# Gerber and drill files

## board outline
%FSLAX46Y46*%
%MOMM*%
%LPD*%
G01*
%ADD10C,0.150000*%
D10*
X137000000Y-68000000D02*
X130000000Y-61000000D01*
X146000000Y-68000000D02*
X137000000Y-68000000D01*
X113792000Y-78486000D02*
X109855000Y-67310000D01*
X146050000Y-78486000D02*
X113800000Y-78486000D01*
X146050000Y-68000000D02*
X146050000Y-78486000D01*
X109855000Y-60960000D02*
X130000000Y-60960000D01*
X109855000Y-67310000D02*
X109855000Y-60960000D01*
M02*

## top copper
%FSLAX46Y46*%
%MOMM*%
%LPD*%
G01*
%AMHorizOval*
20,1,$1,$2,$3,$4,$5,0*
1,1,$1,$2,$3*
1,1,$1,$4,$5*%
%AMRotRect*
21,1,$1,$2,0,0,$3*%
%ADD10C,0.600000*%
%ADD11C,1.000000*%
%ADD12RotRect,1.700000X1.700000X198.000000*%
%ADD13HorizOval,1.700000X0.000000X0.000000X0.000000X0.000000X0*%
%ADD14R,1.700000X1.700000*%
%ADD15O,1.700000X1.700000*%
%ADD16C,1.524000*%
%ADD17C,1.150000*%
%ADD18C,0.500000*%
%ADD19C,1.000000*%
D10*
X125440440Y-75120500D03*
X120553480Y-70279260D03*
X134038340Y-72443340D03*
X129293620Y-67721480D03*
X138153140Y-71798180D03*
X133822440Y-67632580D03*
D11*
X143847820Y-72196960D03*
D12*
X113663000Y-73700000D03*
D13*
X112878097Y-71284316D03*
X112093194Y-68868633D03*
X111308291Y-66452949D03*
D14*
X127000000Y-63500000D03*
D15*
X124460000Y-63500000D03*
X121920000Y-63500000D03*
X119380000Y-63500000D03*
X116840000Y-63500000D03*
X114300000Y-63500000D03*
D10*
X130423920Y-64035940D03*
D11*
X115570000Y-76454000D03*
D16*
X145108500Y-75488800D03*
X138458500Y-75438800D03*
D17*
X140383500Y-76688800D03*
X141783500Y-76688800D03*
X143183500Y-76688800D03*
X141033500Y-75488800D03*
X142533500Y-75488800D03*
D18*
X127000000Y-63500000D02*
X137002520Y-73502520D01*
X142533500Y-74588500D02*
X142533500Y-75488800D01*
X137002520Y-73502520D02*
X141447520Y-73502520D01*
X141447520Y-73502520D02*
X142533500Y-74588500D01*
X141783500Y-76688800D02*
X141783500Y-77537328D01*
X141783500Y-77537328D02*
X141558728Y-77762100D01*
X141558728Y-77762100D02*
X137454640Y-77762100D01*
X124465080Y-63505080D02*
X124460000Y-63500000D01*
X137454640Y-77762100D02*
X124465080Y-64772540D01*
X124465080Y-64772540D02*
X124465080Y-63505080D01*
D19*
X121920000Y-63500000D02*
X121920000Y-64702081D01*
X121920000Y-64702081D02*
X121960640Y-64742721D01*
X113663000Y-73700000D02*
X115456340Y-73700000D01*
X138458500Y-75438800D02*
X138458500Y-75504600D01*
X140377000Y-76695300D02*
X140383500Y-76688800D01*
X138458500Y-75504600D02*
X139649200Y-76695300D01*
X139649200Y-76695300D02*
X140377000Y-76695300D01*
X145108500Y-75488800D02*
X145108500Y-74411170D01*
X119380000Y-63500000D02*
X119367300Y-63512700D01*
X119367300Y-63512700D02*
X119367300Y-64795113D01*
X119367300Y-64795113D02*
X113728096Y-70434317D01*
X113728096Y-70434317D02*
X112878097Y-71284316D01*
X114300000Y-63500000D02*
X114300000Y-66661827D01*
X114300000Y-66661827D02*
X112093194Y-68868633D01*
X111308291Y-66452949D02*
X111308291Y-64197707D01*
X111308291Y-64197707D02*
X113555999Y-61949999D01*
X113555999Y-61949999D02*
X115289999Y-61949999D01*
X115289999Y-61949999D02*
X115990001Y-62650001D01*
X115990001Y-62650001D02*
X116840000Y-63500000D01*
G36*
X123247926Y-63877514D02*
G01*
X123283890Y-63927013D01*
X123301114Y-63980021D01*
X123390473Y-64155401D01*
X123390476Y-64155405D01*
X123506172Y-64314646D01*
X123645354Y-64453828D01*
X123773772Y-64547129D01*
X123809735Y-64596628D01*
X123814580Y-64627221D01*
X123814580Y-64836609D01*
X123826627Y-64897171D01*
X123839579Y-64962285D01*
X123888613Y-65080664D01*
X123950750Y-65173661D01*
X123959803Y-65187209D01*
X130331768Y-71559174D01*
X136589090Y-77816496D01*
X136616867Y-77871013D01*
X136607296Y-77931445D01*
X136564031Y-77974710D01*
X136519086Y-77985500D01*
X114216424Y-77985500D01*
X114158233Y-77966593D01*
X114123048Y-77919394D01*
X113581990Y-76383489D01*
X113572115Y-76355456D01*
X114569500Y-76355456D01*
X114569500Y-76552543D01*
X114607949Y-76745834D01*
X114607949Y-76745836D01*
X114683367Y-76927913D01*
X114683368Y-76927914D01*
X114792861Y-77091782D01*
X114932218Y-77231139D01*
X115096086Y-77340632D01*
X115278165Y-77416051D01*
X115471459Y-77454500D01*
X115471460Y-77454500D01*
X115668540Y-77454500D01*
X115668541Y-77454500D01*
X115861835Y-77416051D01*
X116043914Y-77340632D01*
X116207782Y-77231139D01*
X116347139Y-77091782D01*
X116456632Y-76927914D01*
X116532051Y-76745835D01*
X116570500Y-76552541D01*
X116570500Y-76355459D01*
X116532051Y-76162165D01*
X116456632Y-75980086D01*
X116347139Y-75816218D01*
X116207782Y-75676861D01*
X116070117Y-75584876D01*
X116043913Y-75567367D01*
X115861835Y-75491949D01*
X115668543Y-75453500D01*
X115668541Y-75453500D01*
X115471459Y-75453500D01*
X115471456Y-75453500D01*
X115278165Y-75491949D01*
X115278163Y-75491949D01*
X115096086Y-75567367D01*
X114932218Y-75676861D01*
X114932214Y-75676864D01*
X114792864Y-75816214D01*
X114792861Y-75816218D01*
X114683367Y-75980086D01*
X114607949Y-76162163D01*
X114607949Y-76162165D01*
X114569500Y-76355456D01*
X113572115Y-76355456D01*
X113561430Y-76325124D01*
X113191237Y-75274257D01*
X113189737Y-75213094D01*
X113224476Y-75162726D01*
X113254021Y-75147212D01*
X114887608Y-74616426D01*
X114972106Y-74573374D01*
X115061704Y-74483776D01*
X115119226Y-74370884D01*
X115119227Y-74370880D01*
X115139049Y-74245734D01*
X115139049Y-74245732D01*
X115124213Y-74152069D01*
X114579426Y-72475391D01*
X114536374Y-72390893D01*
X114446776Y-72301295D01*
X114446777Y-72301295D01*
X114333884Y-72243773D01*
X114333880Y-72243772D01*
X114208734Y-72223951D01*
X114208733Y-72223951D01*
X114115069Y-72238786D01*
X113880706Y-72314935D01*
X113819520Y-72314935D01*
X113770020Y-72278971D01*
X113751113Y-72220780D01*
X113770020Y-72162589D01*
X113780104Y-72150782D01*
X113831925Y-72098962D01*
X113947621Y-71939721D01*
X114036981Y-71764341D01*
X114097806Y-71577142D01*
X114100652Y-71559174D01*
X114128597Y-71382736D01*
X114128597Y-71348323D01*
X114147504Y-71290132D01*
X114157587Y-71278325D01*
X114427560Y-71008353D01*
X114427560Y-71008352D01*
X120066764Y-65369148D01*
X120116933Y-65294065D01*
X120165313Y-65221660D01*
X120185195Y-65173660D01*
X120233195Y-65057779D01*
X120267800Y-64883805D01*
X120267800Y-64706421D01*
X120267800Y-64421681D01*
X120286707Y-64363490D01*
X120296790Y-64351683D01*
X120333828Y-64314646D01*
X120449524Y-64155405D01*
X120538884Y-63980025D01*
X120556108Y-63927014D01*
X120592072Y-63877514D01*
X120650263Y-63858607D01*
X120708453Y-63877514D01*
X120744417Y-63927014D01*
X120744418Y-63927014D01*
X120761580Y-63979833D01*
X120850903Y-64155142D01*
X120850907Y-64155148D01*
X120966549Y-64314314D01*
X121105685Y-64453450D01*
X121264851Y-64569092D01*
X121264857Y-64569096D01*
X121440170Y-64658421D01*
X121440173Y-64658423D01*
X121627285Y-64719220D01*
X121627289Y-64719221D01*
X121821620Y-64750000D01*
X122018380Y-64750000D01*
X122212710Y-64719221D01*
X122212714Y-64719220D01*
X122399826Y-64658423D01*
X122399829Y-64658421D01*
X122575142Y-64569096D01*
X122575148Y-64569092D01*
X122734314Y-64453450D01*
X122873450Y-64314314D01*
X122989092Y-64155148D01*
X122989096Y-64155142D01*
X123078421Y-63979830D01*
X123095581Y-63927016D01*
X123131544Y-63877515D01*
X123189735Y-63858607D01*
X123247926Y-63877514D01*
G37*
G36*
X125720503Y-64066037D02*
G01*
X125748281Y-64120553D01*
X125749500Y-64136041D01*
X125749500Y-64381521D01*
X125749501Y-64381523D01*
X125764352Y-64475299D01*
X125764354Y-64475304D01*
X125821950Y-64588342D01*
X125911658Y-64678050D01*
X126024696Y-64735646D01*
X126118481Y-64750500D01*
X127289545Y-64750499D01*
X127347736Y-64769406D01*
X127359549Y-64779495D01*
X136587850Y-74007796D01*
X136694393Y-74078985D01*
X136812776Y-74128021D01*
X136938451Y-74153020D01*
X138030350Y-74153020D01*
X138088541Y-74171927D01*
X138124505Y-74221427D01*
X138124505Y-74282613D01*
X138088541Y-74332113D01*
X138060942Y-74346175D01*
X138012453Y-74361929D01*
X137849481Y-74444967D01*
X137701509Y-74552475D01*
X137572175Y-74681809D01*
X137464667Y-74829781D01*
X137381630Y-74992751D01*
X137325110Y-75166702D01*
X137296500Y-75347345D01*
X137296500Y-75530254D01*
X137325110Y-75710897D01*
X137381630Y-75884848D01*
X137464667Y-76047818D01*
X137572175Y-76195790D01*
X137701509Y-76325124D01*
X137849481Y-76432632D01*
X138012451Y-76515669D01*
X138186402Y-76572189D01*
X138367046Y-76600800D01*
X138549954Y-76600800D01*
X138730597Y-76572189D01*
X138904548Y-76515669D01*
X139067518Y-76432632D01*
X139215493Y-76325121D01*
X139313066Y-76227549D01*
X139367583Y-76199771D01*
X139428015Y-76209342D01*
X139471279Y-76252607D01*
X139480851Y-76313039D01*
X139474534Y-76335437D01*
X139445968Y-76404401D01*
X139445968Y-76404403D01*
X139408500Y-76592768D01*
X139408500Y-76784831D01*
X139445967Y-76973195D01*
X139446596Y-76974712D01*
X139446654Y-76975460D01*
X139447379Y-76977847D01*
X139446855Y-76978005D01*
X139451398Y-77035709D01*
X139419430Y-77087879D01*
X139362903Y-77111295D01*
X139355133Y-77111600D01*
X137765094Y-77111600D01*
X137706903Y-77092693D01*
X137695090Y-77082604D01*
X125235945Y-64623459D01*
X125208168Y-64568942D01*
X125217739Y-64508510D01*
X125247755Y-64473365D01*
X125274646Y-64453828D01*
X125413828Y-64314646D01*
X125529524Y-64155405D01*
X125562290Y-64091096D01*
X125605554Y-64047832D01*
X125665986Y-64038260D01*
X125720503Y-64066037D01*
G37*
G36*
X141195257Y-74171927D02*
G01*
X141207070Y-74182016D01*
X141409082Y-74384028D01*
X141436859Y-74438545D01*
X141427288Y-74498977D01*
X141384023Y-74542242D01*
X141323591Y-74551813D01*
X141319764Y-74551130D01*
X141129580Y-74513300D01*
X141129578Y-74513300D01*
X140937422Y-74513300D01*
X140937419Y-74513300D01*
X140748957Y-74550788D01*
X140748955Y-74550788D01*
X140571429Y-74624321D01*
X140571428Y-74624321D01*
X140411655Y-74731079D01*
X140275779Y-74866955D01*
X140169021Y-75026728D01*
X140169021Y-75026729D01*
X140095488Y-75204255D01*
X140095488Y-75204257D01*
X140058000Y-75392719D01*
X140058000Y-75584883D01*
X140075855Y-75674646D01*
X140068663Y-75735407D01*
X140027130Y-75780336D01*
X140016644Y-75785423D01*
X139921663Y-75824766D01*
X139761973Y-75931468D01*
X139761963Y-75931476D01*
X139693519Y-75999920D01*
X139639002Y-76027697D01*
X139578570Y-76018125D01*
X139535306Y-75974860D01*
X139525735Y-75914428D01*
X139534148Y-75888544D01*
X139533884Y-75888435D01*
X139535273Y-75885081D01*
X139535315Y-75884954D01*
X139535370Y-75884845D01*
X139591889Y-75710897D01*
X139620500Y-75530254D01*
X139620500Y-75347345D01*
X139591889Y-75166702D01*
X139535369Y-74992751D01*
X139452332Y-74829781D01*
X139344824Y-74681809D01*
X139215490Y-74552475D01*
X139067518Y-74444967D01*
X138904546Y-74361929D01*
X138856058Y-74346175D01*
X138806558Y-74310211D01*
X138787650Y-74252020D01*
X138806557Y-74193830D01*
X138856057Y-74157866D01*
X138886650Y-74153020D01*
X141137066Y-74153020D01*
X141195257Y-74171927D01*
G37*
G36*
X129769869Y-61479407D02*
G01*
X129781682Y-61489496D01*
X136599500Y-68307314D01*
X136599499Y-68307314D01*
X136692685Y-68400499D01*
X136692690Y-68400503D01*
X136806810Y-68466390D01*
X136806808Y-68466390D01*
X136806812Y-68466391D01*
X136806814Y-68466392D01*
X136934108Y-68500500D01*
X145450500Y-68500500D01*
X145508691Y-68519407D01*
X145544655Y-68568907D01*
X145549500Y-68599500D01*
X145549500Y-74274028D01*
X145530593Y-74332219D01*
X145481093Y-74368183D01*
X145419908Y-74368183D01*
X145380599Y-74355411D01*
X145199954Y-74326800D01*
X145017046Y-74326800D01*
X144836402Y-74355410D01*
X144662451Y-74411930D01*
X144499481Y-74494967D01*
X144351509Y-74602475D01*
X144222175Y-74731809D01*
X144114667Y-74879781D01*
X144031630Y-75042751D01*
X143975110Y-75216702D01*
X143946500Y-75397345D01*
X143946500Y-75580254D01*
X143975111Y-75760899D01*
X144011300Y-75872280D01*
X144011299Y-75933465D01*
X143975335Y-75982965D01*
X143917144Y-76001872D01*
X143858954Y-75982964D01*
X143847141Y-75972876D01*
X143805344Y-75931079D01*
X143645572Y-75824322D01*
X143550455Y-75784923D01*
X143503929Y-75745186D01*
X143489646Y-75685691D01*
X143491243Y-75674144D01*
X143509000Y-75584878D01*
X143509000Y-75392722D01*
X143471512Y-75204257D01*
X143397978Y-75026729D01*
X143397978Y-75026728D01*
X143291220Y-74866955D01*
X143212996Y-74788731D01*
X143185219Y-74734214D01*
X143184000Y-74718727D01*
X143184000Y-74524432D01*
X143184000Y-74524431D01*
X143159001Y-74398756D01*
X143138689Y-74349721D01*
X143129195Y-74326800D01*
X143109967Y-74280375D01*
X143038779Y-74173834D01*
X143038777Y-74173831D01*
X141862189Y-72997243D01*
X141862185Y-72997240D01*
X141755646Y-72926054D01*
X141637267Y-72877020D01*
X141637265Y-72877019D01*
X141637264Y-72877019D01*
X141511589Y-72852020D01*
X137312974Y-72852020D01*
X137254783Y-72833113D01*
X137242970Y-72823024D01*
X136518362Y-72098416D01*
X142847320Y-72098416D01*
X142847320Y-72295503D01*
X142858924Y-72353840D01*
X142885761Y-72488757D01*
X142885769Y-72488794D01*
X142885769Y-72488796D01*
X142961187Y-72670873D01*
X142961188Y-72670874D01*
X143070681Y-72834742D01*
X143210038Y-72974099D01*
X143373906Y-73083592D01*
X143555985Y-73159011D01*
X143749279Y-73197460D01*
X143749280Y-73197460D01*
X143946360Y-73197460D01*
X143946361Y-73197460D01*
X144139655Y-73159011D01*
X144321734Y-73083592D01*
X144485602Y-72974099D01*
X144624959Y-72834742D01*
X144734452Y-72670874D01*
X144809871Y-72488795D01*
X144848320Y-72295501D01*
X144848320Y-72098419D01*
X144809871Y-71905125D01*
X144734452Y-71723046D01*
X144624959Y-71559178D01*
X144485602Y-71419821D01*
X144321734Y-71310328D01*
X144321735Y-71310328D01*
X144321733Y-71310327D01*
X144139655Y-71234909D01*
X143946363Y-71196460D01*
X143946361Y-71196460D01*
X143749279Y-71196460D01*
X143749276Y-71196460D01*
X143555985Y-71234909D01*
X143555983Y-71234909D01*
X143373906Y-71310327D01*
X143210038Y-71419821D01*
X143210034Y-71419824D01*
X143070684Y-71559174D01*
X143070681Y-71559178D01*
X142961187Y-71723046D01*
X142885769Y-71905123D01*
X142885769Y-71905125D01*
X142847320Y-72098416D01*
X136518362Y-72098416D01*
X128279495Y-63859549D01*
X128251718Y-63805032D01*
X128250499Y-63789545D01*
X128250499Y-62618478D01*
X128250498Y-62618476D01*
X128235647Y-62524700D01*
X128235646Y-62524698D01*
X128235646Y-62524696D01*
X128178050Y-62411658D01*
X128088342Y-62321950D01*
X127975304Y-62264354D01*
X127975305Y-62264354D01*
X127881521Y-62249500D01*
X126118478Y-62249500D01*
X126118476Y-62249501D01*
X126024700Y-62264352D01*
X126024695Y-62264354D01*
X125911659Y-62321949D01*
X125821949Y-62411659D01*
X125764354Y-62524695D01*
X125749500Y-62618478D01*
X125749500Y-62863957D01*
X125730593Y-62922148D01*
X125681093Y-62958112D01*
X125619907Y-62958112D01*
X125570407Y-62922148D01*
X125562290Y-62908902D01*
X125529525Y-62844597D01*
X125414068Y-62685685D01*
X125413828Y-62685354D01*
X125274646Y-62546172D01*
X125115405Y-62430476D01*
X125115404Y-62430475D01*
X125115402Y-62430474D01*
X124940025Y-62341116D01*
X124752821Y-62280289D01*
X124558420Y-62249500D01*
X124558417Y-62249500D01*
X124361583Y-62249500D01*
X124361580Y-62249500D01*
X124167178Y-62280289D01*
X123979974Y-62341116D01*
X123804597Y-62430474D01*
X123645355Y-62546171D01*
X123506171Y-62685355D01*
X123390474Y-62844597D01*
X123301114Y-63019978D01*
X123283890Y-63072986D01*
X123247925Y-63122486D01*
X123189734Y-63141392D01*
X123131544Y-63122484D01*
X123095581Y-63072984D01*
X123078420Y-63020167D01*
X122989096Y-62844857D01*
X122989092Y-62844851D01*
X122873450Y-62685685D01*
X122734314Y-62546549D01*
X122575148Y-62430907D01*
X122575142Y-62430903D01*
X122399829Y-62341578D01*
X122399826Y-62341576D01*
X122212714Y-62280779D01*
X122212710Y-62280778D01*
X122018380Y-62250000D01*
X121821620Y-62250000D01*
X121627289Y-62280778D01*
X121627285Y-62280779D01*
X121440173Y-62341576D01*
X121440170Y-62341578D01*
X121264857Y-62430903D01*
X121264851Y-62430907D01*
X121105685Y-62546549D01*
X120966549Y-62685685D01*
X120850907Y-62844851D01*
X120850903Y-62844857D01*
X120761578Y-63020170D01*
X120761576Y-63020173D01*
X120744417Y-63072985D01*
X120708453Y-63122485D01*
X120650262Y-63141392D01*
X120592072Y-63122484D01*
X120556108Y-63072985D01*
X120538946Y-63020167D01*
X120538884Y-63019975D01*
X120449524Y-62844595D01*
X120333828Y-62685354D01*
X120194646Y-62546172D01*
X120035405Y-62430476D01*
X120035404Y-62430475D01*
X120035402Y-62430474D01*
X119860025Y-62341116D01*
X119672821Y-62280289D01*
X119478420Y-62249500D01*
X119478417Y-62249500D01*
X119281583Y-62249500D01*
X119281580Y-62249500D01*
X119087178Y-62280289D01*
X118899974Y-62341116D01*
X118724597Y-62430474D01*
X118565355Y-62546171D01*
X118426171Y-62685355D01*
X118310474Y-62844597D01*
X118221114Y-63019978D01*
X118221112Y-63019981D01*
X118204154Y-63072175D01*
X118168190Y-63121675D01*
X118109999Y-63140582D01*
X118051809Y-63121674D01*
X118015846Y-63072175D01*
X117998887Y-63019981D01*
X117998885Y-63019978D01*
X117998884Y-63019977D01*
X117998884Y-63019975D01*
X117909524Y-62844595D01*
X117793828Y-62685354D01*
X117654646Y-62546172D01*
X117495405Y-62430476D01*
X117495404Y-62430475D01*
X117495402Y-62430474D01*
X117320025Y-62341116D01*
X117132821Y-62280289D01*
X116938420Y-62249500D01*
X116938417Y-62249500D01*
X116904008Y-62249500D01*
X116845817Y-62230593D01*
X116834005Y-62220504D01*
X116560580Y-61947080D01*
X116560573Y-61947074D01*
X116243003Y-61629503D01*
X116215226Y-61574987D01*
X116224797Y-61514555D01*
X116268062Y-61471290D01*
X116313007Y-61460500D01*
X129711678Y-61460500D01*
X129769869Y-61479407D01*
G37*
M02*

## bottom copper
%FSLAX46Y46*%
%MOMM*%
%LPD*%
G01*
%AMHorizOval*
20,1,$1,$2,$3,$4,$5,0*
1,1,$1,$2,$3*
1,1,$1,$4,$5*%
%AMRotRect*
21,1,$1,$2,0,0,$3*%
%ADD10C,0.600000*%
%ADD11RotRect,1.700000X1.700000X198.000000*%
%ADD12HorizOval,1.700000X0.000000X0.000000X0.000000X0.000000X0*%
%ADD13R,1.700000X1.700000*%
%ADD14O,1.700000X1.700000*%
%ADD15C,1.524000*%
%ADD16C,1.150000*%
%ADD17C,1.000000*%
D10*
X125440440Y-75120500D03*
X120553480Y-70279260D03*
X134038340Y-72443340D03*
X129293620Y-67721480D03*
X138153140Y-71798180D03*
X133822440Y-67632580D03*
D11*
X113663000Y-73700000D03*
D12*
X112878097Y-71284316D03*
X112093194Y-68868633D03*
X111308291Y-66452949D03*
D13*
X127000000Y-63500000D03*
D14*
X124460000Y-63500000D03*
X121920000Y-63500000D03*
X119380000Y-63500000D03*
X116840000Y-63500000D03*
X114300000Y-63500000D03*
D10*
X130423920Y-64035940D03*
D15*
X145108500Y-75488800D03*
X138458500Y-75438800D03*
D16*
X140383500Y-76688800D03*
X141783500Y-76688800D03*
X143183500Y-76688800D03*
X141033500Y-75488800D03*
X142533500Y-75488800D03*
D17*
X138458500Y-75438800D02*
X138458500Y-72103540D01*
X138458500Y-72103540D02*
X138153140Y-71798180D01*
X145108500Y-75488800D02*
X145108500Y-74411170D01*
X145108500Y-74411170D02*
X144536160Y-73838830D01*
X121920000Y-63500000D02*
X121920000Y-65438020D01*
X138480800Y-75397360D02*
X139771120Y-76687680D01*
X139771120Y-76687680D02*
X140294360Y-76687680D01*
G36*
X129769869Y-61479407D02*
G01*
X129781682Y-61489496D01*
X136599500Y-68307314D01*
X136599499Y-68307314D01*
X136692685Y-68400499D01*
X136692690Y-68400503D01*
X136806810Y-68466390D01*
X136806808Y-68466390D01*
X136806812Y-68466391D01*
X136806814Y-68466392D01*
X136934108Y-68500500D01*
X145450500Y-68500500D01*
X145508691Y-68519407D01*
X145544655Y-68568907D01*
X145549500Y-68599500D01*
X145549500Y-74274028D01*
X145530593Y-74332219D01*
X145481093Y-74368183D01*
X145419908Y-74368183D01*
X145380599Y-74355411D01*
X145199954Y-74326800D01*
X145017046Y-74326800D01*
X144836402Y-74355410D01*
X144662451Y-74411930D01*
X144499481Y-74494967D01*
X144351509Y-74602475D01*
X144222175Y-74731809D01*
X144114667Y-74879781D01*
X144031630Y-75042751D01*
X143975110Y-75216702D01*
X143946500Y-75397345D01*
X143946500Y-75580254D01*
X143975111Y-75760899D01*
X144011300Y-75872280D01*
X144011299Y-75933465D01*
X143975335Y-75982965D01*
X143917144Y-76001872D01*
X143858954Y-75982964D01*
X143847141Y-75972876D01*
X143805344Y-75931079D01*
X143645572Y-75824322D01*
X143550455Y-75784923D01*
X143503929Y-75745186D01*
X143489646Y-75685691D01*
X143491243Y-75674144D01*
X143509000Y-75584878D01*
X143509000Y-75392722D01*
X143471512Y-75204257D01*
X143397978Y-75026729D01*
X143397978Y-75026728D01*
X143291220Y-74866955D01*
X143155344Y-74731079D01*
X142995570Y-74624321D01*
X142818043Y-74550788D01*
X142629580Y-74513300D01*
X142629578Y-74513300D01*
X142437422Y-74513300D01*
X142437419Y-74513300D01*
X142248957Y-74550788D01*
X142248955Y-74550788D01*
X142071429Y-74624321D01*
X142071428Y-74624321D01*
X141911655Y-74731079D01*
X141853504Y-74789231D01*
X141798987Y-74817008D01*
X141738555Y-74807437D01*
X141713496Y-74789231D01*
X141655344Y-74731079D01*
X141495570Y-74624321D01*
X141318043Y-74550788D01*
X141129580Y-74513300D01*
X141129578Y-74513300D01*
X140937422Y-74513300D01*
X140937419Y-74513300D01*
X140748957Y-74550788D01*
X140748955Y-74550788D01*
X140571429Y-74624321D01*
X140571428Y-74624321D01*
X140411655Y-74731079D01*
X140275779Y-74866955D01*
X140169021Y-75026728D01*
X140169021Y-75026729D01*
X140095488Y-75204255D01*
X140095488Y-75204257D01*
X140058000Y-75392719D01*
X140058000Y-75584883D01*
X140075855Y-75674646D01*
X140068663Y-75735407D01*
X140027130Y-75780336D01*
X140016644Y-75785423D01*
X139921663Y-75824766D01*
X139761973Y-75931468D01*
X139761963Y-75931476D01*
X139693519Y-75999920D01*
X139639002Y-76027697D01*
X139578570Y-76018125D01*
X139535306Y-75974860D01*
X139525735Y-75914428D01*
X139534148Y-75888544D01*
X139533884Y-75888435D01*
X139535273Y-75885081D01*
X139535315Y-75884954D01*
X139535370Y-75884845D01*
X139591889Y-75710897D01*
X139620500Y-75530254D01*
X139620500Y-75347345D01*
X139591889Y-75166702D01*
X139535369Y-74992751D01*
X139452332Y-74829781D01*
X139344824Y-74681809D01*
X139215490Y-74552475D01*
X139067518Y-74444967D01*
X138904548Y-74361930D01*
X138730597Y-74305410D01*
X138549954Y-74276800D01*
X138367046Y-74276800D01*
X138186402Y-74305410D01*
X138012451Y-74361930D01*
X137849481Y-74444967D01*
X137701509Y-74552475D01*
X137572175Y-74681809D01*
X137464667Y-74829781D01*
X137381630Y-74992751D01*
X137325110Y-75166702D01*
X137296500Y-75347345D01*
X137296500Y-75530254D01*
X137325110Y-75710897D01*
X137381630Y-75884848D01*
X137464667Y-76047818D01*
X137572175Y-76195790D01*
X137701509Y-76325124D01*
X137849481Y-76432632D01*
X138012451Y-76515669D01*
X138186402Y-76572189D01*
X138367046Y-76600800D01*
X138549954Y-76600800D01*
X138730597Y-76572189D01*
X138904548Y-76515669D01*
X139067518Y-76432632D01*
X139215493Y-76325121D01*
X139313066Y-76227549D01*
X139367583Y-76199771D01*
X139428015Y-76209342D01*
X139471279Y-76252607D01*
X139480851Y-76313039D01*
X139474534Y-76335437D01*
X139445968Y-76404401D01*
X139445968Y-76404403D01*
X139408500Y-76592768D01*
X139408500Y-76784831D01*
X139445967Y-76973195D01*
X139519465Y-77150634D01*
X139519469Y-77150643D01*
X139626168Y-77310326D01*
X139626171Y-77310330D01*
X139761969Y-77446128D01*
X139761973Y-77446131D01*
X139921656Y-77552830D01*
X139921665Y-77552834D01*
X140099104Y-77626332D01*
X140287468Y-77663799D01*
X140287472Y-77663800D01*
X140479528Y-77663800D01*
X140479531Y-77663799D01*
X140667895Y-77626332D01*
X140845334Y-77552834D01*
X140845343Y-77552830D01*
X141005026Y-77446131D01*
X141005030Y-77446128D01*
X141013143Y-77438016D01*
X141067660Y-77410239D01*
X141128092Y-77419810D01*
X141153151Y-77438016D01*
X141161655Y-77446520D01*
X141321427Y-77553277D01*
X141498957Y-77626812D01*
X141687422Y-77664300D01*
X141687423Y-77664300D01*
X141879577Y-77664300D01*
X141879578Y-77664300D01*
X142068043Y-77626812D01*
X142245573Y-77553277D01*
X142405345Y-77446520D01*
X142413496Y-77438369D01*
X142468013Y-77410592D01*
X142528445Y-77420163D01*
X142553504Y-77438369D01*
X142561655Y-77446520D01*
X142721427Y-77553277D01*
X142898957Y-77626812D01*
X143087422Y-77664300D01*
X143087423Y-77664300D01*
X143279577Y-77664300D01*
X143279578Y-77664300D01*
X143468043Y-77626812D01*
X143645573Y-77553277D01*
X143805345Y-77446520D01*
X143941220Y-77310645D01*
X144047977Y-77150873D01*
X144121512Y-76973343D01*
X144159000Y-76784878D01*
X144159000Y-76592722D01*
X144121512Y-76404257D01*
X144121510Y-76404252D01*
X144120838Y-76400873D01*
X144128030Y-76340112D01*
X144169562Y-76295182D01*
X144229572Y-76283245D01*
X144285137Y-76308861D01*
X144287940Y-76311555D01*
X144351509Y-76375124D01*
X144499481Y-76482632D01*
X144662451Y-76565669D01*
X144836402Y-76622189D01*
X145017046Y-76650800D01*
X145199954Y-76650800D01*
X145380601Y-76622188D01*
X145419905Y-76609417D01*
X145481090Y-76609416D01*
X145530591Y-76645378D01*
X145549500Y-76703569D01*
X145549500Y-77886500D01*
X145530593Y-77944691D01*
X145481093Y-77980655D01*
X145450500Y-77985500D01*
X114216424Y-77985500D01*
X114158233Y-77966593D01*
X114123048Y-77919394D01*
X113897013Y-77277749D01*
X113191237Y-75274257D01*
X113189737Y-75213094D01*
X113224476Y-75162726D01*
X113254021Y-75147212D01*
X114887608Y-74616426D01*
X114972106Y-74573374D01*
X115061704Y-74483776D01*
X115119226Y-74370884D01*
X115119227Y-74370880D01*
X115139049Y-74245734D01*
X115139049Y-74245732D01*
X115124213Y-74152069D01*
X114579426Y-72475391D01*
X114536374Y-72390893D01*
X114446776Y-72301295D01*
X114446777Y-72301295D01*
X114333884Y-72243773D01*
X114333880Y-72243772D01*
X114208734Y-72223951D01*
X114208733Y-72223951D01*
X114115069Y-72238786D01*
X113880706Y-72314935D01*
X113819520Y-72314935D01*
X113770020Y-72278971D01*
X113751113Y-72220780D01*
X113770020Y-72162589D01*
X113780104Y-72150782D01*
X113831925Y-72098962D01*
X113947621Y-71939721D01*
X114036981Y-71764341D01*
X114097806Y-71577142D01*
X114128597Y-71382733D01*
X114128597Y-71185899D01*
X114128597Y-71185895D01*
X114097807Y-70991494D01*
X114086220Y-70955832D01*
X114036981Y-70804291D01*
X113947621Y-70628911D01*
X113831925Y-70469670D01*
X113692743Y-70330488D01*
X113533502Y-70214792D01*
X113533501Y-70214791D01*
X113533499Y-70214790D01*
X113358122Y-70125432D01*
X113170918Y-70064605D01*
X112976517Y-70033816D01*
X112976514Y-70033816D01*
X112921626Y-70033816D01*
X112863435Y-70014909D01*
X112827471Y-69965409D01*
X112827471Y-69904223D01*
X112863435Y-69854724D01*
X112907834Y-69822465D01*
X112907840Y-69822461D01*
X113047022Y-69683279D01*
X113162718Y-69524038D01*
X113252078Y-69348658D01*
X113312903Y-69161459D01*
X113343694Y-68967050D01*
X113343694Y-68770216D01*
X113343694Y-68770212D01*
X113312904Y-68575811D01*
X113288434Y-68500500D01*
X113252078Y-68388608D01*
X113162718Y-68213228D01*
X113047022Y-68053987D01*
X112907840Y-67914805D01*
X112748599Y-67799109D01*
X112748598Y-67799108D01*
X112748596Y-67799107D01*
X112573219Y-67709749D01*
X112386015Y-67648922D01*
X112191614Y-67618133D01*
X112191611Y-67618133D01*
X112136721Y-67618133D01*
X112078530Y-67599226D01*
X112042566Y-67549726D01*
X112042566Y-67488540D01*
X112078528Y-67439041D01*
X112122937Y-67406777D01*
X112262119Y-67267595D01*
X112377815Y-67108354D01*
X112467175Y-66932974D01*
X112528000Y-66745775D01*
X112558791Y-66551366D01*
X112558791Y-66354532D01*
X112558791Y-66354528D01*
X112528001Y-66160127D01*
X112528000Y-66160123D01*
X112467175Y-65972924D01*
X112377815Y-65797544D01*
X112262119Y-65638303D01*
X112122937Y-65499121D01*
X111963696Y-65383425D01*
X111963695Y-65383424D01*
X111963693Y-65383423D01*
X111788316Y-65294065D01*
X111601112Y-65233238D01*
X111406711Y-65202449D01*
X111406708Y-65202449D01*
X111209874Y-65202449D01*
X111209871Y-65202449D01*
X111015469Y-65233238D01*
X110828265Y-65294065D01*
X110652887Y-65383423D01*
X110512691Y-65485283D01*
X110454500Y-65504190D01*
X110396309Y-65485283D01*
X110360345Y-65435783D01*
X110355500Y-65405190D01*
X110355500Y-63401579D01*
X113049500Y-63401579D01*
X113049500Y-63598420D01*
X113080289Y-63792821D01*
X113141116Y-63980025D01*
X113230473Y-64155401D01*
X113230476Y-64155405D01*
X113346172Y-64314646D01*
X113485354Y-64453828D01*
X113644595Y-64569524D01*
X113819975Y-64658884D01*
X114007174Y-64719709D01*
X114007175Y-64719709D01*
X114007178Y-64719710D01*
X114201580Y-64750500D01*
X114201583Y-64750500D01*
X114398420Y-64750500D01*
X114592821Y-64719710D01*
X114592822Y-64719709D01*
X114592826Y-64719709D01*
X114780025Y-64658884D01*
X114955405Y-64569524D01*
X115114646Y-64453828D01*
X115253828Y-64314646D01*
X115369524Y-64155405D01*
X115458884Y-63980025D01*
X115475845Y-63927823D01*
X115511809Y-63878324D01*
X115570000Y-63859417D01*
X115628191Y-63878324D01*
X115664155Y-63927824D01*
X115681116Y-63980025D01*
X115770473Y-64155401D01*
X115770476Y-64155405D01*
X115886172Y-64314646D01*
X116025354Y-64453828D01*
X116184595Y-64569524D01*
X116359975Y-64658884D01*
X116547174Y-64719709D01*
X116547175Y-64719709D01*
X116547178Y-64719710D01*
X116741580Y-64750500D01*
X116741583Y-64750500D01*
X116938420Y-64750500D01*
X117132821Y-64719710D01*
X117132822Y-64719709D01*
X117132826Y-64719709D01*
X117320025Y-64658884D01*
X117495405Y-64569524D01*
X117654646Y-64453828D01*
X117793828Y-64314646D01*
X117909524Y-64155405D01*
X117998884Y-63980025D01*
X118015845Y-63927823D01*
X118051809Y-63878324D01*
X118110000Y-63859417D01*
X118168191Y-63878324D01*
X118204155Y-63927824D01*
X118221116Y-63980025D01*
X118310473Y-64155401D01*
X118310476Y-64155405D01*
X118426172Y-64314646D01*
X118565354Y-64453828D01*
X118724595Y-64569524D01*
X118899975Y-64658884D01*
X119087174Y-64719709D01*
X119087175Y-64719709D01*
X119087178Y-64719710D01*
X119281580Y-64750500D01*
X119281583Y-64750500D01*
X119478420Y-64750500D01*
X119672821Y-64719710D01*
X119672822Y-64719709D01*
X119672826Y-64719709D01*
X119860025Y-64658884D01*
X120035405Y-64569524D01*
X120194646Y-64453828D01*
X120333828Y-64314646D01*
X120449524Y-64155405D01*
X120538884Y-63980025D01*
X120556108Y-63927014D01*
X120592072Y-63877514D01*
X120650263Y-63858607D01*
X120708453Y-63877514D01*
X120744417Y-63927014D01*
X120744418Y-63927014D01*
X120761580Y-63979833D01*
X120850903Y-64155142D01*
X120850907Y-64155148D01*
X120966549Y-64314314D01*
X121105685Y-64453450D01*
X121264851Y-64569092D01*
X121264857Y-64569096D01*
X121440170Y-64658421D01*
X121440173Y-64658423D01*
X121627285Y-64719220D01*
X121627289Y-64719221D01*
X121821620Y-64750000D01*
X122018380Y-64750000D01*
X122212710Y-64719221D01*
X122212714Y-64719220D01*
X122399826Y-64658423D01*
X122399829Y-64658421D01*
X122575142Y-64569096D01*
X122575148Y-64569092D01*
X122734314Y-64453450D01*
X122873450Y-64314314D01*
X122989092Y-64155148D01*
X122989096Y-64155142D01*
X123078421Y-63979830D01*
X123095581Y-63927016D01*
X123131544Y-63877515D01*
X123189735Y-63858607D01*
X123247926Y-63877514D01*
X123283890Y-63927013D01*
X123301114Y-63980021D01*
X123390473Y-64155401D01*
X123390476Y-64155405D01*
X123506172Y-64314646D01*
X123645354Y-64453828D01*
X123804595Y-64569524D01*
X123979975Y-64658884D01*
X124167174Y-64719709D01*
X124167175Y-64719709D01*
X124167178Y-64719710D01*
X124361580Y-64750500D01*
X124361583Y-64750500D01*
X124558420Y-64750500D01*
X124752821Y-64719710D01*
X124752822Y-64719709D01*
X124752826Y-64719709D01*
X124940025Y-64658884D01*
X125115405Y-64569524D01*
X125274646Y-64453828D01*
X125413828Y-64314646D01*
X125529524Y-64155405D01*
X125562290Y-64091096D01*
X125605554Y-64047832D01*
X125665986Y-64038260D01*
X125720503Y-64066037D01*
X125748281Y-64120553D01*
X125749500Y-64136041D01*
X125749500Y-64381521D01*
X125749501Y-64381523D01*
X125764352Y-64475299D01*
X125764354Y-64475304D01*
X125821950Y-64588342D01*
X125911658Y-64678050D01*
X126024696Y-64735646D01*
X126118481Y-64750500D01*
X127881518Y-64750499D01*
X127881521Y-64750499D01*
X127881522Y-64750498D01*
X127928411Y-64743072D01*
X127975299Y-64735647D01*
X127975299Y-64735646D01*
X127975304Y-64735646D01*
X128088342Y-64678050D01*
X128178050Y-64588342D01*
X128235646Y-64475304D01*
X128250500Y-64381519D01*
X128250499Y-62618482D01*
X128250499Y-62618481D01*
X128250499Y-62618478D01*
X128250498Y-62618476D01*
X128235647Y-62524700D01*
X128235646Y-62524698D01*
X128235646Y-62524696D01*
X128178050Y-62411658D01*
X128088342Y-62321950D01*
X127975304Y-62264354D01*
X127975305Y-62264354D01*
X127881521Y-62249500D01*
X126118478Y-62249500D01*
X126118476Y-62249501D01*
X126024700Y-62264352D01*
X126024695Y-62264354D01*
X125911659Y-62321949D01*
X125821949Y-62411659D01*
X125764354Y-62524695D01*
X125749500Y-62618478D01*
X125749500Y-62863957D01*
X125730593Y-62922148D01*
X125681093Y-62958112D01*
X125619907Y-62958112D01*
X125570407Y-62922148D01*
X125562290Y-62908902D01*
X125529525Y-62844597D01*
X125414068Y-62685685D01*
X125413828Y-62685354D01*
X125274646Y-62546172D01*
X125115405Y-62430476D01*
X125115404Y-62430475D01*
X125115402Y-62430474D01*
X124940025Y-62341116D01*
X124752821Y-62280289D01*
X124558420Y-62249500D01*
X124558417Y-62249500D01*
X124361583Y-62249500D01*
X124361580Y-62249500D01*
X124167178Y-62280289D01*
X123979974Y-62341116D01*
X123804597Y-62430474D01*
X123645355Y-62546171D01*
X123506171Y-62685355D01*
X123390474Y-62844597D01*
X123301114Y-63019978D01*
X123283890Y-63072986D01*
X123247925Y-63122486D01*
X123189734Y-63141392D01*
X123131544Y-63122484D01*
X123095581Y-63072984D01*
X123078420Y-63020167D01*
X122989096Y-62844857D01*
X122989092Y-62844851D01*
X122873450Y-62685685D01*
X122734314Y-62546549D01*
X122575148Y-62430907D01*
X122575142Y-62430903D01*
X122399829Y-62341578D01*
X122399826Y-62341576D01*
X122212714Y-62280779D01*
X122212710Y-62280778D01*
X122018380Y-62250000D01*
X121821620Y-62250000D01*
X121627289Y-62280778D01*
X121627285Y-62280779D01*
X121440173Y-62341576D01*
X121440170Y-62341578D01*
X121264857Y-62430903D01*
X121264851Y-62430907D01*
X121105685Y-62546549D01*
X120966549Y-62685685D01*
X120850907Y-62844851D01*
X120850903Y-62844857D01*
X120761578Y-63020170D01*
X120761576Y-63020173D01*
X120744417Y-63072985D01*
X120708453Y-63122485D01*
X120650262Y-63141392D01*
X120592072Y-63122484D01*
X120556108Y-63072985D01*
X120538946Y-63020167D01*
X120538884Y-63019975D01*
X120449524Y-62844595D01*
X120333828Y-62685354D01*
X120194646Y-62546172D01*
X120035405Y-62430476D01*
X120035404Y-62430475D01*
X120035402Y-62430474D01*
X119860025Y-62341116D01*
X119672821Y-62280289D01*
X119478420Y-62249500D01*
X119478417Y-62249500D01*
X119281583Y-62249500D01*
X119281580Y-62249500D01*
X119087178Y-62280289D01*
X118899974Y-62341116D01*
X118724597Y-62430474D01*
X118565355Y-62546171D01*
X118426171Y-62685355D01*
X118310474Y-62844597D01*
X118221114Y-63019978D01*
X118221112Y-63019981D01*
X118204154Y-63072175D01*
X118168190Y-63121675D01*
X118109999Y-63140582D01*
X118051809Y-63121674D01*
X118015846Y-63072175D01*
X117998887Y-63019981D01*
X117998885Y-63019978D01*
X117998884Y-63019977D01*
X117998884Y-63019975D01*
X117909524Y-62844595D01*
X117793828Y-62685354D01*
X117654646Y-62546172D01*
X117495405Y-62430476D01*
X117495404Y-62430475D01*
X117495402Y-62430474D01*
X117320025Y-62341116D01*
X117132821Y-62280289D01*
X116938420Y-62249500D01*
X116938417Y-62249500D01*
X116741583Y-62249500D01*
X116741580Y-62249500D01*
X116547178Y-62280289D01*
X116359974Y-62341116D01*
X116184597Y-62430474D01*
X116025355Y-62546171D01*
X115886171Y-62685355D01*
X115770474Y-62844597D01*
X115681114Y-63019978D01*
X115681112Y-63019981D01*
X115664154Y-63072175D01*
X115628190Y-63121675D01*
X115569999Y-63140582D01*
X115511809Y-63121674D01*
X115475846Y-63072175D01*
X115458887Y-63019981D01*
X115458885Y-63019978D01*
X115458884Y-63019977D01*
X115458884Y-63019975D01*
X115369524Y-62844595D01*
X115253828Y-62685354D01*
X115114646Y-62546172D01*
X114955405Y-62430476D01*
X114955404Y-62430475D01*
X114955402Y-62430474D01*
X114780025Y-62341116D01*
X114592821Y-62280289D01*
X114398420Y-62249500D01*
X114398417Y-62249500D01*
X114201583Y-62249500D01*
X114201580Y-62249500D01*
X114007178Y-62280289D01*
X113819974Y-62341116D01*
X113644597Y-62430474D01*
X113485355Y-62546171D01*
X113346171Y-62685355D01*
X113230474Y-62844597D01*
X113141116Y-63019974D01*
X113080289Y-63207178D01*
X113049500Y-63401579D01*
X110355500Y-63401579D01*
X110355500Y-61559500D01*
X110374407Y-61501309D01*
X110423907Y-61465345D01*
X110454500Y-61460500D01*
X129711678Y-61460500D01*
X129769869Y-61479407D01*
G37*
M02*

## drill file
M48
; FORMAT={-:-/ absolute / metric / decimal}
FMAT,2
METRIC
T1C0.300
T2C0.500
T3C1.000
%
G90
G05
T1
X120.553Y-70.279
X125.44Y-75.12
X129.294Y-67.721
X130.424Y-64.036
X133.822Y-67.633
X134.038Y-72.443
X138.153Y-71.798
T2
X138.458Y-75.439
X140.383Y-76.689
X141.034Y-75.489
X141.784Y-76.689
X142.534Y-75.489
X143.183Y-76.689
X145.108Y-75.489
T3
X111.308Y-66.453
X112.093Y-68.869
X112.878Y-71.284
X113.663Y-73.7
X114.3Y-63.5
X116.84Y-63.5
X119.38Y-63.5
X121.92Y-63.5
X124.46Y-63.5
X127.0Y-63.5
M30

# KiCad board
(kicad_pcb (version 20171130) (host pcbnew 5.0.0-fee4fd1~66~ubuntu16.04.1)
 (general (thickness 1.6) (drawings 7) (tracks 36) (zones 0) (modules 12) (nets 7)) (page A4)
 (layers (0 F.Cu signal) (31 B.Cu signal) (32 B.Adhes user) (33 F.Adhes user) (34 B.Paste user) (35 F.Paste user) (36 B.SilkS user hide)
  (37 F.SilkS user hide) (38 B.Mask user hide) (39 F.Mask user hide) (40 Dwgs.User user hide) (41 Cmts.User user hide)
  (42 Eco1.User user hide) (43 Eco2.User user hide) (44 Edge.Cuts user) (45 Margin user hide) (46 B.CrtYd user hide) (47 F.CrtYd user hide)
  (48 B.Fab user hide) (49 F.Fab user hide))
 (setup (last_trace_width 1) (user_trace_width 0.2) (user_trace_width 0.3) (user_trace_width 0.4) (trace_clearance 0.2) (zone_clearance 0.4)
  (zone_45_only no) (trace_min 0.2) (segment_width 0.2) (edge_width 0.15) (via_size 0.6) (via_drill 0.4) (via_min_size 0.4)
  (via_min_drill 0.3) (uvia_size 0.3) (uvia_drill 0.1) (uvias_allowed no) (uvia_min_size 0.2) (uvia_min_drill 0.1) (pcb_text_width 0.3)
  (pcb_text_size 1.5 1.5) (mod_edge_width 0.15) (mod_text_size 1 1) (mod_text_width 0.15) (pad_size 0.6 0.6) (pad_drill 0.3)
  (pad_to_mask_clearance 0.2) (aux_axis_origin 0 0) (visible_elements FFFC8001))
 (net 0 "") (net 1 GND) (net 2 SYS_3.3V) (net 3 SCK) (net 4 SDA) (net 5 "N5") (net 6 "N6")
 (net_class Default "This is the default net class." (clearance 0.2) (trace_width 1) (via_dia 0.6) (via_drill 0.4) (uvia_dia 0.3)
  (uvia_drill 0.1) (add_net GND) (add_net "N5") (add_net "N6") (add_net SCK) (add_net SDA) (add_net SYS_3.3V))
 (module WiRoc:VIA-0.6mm (layer F.Cu) (at 125.44044 75.1205)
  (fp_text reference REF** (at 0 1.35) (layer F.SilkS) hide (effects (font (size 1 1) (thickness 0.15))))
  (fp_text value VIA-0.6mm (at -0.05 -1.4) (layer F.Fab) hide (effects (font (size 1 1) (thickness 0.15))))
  (pad 1 thru_hole circle (at 0 0) (size 0.6 0.6) (drill 0.3) (layers *.Cu) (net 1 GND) (zone_connect 2)))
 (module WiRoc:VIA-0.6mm (layer F.Cu) (at 120.55348 70.27926)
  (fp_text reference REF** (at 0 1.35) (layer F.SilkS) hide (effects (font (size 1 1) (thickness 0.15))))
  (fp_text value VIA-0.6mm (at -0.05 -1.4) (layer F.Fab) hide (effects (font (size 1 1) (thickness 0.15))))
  (pad 1 thru_hole circle (at 0 0) (size 0.6 0.6) (drill 0.3) (layers *.Cu) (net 1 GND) (zone_connect 2)))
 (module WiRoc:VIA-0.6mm (layer F.Cu) (at 134.03834 72.44334)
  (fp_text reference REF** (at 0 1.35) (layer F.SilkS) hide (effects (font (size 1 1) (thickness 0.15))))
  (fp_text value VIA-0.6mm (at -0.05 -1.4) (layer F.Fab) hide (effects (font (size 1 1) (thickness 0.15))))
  (pad 1 thru_hole circle (at 0 0) (size 0.6 0.6) (drill 0.3) (layers *.Cu) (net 1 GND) (zone_connect 2)))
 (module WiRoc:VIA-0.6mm (layer F.Cu) (at 129.29362 67.72148)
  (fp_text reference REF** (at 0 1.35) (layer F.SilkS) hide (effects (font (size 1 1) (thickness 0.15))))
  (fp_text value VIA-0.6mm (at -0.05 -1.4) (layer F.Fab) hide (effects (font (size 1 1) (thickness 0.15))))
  (pad 1 thru_hole circle (at 0 0) (size 0.6 0.6) (drill 0.3) (layers *.Cu) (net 1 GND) (zone_connect 2)))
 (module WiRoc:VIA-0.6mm (layer F.Cu) (at 138.15314 71.79818)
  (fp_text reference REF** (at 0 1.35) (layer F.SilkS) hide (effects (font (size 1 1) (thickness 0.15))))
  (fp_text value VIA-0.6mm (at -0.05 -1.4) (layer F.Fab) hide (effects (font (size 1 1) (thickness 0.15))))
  (pad 1 thru_hole circle (at 0 0) (size 0.6 0.6) (drill 0.3) (layers *.Cu) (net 1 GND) (zone_connect 2)))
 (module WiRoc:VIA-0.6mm (layer F.Cu) (at 133.82244 67.63258)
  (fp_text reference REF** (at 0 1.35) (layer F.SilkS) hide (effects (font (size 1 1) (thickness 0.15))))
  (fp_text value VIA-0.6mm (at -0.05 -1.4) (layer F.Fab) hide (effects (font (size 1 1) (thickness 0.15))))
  (pad 1 thru_hole circle (at 0 0) (size 0.6 0.6) (drill 0.3) (layers *.Cu) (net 1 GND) (zone_connect 2)))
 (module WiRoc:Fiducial (layer F.Cu) (at 143.84782 72.19696)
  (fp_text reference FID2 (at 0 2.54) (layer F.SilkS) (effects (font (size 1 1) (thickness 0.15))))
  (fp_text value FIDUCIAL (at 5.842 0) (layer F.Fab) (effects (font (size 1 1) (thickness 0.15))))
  (pad 1 smd circle (at 0 0) (size 1 1) (layers F.Cu F.Mask) (solder_mask_margin 0.5) (clearance 0.5)))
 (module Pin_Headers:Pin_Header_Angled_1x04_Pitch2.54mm (layer F.Cu) (at 113.663 73.7 198)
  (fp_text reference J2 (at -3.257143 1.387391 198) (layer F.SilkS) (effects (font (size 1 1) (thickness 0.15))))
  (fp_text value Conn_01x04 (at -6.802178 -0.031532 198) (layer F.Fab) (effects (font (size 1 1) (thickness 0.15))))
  (pad 1 thru_hole rect (at 0 0 198) (size 1.7 1.7) (drill 1) (layers *.Cu *.Mask) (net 1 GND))
  (pad 2 thru_hole oval (at 0 2.54 198) (size 1.7 1.7) (drill 1) (layers *.Cu *.Mask) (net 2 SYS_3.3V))
  (pad 3 thru_hole oval (at 0 5.08 198) (size 1.7 1.7) (drill 1) (layers *.Cu *.Mask) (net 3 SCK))
  (pad 4 thru_hole oval (at -0.000001 7.62 198) (size 1.7 1.7) (drill 1) (layers *.Cu *.Mask) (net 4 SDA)))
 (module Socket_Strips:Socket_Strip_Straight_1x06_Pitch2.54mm (layer F.Cu) (at 127 63.5 270)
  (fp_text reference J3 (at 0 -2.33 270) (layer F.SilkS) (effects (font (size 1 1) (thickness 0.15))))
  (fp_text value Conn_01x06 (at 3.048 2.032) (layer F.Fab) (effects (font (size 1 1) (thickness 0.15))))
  (pad 1 thru_hole rect (at 0 0 270) (size 1.7 1.7) (drill 1) (layers *.Cu *.Mask) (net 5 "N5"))
  (pad 2 thru_hole oval (at 0 2.54 270) (size 1.7 1.7) (drill 1) (layers *.Cu *.Mask) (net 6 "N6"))
  (pad 3 thru_hole oval (at 0 5.08 270) (size 1.7 1.7) (drill 1) (layers *.Cu *.Mask) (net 1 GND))
  (pad 4 thru_hole oval (at 0 7.62 270) (size 1.7 1.7) (drill 1) (layers *.Cu *.Mask) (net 2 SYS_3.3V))
  (pad 5 thru_hole oval (at 0 10.16 270) (size 1.7 1.7) (drill 1) (layers *.Cu *.Mask) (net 4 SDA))
  (pad 6 thru_hole oval (at 0 12.7 270) (size 1.7 1.7) (drill 1) (layers *.Cu *.Mask) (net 3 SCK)))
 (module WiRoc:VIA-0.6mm (layer F.Cu) (at 130.42392 64.03594)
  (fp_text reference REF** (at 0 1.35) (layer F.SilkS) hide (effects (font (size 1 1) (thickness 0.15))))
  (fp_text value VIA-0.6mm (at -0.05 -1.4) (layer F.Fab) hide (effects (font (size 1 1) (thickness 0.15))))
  (pad 1 thru_hole circle (at 0 0) (size 0.6 0.6) (drill 0.3) (layers *.Cu) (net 1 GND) (zone_connect 2)))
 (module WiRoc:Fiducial (layer F.Cu) (at 115.57 76.454)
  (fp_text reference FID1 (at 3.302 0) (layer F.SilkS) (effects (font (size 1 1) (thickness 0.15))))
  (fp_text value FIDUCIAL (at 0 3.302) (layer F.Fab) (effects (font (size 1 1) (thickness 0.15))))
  (pad 1 smd circle (at 0 0) (size 1 1) (layers F.Cu F.Mask) (solder_mask_margin 0.5) (clearance 0.5)))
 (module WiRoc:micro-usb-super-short (layer F.Cu) (at 141.7835 75.4888 180)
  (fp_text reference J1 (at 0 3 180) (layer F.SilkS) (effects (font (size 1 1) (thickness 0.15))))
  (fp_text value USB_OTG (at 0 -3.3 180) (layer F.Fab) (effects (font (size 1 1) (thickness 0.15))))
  (pad 6 thru_hole circle (at -3.325 0 180) (size 1.524 1.524) (drill 0.5) (layers *.Cu *.Mask) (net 1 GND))
  (pad 6 thru_hole circle (at 3.325 0.05 180) (size 1.524 1.524) (drill 0.5) (layers *.Cu *.Mask) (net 1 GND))
  (pad 5 thru_hole circle (at 1.4 -1.2 180) (size 1.15 1.15) (drill 0.5) (layers *.Cu *.Mask) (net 1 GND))
  (pad 3 thru_hole circle (at 0 -1.2 180) (size 1.15 1.15) (drill 0.5) (layers *.Cu *.Mask) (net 6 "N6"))
  (pad 1 thru_hole circle (at -1.4 -1.2 180) (size 1.15 1.15) (drill 0.5) (layers *.Cu *.Mask))
  (pad 4 thru_hole circle (at 0.75 0 180) (size 1.15 1.15) (drill 0.5) (layers *.Cu *.Mask))
  (pad 2 thru_hole circle (at -0.75 0 180) (size 1.15 1.15) (drill 0.5) (layers *.Cu *.Mask) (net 5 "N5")))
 (gr_line (start 137 68) (end 130 61) (layer Edge.Cuts) (width 0.15))
 (gr_line (start 146 68) (end 137 68) (layer Edge.Cuts) (width 0.15))
 (gr_line (start 113.792 78.486) (end 109.855 67.31) (layer Edge.Cuts) (width 0.15))
 (gr_line (start 146.05 78.486) (end 113.8 78.486) (layer Edge.Cuts) (width 0.15))
 (gr_line (start 146.05 68) (end 146.05 78.486) (layer Edge.Cuts) (width 0.15))
 (gr_line (start 109.855 60.96) (end 130 60.96) (layer Edge.Cuts) (width 0.15))
 (gr_line (start 109.855 67.31) (end 109.855 60.96) (layer Edge.Cuts) (width 0.15))
 (segment (start 127 63.5) (end 137.00252 73.50252) (width 0.5) (layer F.Cu) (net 5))
 (segment (start 142.5335 74.5885) (end 142.5335 75.4888) (width 0.5) (layer F.Cu) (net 5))
 (segment (start 137.00252 73.50252) (end 141.44752 73.50252) (width 0.5) (layer F.Cu) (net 5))
 (segment (start 141.44752 73.50252) (end 142.5335 74.5885) (width 0.5) (layer F.Cu) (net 5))
 (segment (start 141.7835 76.6888) (end 141.7835 77.537328) (width 0.5) (layer F.Cu) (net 6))
 (segment (start 141.7835 77.537328) (end 141.558728 77.7621) (width 0.5) (layer F.Cu) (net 6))
 (segment (start 141.558728 77.7621) (end 137.45464 77.7621) (width 0.5) (layer F.Cu) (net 6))
 (segment (start 124.46508 63.50508) (end 124.46 63.5) (width 0.5) (layer F.Cu) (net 6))
 (segment (start 137.45464 77.7621) (end 124.46508 64.77254) (width 0.5) (layer F.Cu) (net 6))
 (segment (start 124.46508 64.77254) (end 124.46508 63.50508) (width 0.5) (layer F.Cu) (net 6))
 (segment (start 138.4585 75.4388) (end 138.4585 72.10354) (width 1) (layer B.Cu) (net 1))
 (segment (start 138.4585 72.10354) (end 138.15314 71.79818) (width 1) (layer B.Cu) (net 1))
 (segment (start 145.1085 75.4888) (end 145.1085 74.41117) (width 1) (layer B.Cu) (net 1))
 (segment (start 145.1085 74.41117) (end 144.53616 73.83883) (width 1) (layer B.Cu) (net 1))
 (segment (start 121.92 63.5) (end 121.92 65.43802) (width 1) (layer B.Cu) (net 1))
 (segment (start 121.92 63.5) (end 121.92 64.702081) (width 1) (layer F.Cu) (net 1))
 (segment (start 121.92 64.702081) (end 121.96064 64.742721) (width 1) (layer F.Cu) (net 1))
 (segment (start 113.663 73.7) (end 115.45634 73.7) (width 1) (layer F.Cu) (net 1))
 (segment (start 138.4585 75.4388) (end 138.4585 75.5046) (width 1) (layer F.Cu) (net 1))
 (segment (start 140.377 76.6953) (end 140.3835 76.6888) (width 1) (layer F.Cu) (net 1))
 (segment (start 138.4585 75.5046) (end 139.6492 76.6953) (width 1) (layer F.Cu) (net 1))
 (segment (start 139.6492 76.6953) (end 140.377 76.6953) (width 1) (layer F.Cu) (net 1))
 (segment (start 145.1085 75.4888) (end 145.1085 74.41117) (width 1) (layer F.Cu) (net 1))
 (segment (start 138.4808 75.39736) (end 139.77112 76.68768) (width 1) (layer B.Cu) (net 1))
 (segment (start 139.77112 76.68768) (end 140.29436 76.68768) (width 1) (layer B.Cu) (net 1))
 (segment (start 119.38 63.5) (end 119.3673 63.5127) (width 1) (layer F.Cu) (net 2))
 (segment (start 119.3673 63.5127) (end 119.3673 64.795113) (width 1) (layer F.Cu) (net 2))
 (segment (start 119.3673 64.795113) (end 113.728096 70.434317) (width 1) (layer F.Cu) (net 2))
 (segment (start 113.728096 70.434317) (end 112.878097 71.284316) (width 1) (layer F.Cu) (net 2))
 (segment (start 114.3 63.5) (end 114.3 66.661827) (width 1) (layer F.Cu) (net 3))
 (segment (start 114.3 66.661827) (end 112.093194 68.868633) (width 1) (layer F.Cu) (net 3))
 (segment (start 111.308291 66.452949) (end 111.308291 64.197707) (width 1) (layer F.Cu) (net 4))
 (segment (start 111.308291 64.197707) (end 113.555999 61.949999) (width 1) (layer F.Cu) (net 4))
 (segment (start 113.555999 61.949999) (end 115.289999 61.949999) (width 1) (layer F.Cu) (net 4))
 (segment (start 115.289999 61.949999) (end 115.990001 62.650001) (width 1) (layer F.Cu) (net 4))
 (segment (start 115.990001 62.650001) (end 116.84 63.5) (width 1) (layer F.Cu) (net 4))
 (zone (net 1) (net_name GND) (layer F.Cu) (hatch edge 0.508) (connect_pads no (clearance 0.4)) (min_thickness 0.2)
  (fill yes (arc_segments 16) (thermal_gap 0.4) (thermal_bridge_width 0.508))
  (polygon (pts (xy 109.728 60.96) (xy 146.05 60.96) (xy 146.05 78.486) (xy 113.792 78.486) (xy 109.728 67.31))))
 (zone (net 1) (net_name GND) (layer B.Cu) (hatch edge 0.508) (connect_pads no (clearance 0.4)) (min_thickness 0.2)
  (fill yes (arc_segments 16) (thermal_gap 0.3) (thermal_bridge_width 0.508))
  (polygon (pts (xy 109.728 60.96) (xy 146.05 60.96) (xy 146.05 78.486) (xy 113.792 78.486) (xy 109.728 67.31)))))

